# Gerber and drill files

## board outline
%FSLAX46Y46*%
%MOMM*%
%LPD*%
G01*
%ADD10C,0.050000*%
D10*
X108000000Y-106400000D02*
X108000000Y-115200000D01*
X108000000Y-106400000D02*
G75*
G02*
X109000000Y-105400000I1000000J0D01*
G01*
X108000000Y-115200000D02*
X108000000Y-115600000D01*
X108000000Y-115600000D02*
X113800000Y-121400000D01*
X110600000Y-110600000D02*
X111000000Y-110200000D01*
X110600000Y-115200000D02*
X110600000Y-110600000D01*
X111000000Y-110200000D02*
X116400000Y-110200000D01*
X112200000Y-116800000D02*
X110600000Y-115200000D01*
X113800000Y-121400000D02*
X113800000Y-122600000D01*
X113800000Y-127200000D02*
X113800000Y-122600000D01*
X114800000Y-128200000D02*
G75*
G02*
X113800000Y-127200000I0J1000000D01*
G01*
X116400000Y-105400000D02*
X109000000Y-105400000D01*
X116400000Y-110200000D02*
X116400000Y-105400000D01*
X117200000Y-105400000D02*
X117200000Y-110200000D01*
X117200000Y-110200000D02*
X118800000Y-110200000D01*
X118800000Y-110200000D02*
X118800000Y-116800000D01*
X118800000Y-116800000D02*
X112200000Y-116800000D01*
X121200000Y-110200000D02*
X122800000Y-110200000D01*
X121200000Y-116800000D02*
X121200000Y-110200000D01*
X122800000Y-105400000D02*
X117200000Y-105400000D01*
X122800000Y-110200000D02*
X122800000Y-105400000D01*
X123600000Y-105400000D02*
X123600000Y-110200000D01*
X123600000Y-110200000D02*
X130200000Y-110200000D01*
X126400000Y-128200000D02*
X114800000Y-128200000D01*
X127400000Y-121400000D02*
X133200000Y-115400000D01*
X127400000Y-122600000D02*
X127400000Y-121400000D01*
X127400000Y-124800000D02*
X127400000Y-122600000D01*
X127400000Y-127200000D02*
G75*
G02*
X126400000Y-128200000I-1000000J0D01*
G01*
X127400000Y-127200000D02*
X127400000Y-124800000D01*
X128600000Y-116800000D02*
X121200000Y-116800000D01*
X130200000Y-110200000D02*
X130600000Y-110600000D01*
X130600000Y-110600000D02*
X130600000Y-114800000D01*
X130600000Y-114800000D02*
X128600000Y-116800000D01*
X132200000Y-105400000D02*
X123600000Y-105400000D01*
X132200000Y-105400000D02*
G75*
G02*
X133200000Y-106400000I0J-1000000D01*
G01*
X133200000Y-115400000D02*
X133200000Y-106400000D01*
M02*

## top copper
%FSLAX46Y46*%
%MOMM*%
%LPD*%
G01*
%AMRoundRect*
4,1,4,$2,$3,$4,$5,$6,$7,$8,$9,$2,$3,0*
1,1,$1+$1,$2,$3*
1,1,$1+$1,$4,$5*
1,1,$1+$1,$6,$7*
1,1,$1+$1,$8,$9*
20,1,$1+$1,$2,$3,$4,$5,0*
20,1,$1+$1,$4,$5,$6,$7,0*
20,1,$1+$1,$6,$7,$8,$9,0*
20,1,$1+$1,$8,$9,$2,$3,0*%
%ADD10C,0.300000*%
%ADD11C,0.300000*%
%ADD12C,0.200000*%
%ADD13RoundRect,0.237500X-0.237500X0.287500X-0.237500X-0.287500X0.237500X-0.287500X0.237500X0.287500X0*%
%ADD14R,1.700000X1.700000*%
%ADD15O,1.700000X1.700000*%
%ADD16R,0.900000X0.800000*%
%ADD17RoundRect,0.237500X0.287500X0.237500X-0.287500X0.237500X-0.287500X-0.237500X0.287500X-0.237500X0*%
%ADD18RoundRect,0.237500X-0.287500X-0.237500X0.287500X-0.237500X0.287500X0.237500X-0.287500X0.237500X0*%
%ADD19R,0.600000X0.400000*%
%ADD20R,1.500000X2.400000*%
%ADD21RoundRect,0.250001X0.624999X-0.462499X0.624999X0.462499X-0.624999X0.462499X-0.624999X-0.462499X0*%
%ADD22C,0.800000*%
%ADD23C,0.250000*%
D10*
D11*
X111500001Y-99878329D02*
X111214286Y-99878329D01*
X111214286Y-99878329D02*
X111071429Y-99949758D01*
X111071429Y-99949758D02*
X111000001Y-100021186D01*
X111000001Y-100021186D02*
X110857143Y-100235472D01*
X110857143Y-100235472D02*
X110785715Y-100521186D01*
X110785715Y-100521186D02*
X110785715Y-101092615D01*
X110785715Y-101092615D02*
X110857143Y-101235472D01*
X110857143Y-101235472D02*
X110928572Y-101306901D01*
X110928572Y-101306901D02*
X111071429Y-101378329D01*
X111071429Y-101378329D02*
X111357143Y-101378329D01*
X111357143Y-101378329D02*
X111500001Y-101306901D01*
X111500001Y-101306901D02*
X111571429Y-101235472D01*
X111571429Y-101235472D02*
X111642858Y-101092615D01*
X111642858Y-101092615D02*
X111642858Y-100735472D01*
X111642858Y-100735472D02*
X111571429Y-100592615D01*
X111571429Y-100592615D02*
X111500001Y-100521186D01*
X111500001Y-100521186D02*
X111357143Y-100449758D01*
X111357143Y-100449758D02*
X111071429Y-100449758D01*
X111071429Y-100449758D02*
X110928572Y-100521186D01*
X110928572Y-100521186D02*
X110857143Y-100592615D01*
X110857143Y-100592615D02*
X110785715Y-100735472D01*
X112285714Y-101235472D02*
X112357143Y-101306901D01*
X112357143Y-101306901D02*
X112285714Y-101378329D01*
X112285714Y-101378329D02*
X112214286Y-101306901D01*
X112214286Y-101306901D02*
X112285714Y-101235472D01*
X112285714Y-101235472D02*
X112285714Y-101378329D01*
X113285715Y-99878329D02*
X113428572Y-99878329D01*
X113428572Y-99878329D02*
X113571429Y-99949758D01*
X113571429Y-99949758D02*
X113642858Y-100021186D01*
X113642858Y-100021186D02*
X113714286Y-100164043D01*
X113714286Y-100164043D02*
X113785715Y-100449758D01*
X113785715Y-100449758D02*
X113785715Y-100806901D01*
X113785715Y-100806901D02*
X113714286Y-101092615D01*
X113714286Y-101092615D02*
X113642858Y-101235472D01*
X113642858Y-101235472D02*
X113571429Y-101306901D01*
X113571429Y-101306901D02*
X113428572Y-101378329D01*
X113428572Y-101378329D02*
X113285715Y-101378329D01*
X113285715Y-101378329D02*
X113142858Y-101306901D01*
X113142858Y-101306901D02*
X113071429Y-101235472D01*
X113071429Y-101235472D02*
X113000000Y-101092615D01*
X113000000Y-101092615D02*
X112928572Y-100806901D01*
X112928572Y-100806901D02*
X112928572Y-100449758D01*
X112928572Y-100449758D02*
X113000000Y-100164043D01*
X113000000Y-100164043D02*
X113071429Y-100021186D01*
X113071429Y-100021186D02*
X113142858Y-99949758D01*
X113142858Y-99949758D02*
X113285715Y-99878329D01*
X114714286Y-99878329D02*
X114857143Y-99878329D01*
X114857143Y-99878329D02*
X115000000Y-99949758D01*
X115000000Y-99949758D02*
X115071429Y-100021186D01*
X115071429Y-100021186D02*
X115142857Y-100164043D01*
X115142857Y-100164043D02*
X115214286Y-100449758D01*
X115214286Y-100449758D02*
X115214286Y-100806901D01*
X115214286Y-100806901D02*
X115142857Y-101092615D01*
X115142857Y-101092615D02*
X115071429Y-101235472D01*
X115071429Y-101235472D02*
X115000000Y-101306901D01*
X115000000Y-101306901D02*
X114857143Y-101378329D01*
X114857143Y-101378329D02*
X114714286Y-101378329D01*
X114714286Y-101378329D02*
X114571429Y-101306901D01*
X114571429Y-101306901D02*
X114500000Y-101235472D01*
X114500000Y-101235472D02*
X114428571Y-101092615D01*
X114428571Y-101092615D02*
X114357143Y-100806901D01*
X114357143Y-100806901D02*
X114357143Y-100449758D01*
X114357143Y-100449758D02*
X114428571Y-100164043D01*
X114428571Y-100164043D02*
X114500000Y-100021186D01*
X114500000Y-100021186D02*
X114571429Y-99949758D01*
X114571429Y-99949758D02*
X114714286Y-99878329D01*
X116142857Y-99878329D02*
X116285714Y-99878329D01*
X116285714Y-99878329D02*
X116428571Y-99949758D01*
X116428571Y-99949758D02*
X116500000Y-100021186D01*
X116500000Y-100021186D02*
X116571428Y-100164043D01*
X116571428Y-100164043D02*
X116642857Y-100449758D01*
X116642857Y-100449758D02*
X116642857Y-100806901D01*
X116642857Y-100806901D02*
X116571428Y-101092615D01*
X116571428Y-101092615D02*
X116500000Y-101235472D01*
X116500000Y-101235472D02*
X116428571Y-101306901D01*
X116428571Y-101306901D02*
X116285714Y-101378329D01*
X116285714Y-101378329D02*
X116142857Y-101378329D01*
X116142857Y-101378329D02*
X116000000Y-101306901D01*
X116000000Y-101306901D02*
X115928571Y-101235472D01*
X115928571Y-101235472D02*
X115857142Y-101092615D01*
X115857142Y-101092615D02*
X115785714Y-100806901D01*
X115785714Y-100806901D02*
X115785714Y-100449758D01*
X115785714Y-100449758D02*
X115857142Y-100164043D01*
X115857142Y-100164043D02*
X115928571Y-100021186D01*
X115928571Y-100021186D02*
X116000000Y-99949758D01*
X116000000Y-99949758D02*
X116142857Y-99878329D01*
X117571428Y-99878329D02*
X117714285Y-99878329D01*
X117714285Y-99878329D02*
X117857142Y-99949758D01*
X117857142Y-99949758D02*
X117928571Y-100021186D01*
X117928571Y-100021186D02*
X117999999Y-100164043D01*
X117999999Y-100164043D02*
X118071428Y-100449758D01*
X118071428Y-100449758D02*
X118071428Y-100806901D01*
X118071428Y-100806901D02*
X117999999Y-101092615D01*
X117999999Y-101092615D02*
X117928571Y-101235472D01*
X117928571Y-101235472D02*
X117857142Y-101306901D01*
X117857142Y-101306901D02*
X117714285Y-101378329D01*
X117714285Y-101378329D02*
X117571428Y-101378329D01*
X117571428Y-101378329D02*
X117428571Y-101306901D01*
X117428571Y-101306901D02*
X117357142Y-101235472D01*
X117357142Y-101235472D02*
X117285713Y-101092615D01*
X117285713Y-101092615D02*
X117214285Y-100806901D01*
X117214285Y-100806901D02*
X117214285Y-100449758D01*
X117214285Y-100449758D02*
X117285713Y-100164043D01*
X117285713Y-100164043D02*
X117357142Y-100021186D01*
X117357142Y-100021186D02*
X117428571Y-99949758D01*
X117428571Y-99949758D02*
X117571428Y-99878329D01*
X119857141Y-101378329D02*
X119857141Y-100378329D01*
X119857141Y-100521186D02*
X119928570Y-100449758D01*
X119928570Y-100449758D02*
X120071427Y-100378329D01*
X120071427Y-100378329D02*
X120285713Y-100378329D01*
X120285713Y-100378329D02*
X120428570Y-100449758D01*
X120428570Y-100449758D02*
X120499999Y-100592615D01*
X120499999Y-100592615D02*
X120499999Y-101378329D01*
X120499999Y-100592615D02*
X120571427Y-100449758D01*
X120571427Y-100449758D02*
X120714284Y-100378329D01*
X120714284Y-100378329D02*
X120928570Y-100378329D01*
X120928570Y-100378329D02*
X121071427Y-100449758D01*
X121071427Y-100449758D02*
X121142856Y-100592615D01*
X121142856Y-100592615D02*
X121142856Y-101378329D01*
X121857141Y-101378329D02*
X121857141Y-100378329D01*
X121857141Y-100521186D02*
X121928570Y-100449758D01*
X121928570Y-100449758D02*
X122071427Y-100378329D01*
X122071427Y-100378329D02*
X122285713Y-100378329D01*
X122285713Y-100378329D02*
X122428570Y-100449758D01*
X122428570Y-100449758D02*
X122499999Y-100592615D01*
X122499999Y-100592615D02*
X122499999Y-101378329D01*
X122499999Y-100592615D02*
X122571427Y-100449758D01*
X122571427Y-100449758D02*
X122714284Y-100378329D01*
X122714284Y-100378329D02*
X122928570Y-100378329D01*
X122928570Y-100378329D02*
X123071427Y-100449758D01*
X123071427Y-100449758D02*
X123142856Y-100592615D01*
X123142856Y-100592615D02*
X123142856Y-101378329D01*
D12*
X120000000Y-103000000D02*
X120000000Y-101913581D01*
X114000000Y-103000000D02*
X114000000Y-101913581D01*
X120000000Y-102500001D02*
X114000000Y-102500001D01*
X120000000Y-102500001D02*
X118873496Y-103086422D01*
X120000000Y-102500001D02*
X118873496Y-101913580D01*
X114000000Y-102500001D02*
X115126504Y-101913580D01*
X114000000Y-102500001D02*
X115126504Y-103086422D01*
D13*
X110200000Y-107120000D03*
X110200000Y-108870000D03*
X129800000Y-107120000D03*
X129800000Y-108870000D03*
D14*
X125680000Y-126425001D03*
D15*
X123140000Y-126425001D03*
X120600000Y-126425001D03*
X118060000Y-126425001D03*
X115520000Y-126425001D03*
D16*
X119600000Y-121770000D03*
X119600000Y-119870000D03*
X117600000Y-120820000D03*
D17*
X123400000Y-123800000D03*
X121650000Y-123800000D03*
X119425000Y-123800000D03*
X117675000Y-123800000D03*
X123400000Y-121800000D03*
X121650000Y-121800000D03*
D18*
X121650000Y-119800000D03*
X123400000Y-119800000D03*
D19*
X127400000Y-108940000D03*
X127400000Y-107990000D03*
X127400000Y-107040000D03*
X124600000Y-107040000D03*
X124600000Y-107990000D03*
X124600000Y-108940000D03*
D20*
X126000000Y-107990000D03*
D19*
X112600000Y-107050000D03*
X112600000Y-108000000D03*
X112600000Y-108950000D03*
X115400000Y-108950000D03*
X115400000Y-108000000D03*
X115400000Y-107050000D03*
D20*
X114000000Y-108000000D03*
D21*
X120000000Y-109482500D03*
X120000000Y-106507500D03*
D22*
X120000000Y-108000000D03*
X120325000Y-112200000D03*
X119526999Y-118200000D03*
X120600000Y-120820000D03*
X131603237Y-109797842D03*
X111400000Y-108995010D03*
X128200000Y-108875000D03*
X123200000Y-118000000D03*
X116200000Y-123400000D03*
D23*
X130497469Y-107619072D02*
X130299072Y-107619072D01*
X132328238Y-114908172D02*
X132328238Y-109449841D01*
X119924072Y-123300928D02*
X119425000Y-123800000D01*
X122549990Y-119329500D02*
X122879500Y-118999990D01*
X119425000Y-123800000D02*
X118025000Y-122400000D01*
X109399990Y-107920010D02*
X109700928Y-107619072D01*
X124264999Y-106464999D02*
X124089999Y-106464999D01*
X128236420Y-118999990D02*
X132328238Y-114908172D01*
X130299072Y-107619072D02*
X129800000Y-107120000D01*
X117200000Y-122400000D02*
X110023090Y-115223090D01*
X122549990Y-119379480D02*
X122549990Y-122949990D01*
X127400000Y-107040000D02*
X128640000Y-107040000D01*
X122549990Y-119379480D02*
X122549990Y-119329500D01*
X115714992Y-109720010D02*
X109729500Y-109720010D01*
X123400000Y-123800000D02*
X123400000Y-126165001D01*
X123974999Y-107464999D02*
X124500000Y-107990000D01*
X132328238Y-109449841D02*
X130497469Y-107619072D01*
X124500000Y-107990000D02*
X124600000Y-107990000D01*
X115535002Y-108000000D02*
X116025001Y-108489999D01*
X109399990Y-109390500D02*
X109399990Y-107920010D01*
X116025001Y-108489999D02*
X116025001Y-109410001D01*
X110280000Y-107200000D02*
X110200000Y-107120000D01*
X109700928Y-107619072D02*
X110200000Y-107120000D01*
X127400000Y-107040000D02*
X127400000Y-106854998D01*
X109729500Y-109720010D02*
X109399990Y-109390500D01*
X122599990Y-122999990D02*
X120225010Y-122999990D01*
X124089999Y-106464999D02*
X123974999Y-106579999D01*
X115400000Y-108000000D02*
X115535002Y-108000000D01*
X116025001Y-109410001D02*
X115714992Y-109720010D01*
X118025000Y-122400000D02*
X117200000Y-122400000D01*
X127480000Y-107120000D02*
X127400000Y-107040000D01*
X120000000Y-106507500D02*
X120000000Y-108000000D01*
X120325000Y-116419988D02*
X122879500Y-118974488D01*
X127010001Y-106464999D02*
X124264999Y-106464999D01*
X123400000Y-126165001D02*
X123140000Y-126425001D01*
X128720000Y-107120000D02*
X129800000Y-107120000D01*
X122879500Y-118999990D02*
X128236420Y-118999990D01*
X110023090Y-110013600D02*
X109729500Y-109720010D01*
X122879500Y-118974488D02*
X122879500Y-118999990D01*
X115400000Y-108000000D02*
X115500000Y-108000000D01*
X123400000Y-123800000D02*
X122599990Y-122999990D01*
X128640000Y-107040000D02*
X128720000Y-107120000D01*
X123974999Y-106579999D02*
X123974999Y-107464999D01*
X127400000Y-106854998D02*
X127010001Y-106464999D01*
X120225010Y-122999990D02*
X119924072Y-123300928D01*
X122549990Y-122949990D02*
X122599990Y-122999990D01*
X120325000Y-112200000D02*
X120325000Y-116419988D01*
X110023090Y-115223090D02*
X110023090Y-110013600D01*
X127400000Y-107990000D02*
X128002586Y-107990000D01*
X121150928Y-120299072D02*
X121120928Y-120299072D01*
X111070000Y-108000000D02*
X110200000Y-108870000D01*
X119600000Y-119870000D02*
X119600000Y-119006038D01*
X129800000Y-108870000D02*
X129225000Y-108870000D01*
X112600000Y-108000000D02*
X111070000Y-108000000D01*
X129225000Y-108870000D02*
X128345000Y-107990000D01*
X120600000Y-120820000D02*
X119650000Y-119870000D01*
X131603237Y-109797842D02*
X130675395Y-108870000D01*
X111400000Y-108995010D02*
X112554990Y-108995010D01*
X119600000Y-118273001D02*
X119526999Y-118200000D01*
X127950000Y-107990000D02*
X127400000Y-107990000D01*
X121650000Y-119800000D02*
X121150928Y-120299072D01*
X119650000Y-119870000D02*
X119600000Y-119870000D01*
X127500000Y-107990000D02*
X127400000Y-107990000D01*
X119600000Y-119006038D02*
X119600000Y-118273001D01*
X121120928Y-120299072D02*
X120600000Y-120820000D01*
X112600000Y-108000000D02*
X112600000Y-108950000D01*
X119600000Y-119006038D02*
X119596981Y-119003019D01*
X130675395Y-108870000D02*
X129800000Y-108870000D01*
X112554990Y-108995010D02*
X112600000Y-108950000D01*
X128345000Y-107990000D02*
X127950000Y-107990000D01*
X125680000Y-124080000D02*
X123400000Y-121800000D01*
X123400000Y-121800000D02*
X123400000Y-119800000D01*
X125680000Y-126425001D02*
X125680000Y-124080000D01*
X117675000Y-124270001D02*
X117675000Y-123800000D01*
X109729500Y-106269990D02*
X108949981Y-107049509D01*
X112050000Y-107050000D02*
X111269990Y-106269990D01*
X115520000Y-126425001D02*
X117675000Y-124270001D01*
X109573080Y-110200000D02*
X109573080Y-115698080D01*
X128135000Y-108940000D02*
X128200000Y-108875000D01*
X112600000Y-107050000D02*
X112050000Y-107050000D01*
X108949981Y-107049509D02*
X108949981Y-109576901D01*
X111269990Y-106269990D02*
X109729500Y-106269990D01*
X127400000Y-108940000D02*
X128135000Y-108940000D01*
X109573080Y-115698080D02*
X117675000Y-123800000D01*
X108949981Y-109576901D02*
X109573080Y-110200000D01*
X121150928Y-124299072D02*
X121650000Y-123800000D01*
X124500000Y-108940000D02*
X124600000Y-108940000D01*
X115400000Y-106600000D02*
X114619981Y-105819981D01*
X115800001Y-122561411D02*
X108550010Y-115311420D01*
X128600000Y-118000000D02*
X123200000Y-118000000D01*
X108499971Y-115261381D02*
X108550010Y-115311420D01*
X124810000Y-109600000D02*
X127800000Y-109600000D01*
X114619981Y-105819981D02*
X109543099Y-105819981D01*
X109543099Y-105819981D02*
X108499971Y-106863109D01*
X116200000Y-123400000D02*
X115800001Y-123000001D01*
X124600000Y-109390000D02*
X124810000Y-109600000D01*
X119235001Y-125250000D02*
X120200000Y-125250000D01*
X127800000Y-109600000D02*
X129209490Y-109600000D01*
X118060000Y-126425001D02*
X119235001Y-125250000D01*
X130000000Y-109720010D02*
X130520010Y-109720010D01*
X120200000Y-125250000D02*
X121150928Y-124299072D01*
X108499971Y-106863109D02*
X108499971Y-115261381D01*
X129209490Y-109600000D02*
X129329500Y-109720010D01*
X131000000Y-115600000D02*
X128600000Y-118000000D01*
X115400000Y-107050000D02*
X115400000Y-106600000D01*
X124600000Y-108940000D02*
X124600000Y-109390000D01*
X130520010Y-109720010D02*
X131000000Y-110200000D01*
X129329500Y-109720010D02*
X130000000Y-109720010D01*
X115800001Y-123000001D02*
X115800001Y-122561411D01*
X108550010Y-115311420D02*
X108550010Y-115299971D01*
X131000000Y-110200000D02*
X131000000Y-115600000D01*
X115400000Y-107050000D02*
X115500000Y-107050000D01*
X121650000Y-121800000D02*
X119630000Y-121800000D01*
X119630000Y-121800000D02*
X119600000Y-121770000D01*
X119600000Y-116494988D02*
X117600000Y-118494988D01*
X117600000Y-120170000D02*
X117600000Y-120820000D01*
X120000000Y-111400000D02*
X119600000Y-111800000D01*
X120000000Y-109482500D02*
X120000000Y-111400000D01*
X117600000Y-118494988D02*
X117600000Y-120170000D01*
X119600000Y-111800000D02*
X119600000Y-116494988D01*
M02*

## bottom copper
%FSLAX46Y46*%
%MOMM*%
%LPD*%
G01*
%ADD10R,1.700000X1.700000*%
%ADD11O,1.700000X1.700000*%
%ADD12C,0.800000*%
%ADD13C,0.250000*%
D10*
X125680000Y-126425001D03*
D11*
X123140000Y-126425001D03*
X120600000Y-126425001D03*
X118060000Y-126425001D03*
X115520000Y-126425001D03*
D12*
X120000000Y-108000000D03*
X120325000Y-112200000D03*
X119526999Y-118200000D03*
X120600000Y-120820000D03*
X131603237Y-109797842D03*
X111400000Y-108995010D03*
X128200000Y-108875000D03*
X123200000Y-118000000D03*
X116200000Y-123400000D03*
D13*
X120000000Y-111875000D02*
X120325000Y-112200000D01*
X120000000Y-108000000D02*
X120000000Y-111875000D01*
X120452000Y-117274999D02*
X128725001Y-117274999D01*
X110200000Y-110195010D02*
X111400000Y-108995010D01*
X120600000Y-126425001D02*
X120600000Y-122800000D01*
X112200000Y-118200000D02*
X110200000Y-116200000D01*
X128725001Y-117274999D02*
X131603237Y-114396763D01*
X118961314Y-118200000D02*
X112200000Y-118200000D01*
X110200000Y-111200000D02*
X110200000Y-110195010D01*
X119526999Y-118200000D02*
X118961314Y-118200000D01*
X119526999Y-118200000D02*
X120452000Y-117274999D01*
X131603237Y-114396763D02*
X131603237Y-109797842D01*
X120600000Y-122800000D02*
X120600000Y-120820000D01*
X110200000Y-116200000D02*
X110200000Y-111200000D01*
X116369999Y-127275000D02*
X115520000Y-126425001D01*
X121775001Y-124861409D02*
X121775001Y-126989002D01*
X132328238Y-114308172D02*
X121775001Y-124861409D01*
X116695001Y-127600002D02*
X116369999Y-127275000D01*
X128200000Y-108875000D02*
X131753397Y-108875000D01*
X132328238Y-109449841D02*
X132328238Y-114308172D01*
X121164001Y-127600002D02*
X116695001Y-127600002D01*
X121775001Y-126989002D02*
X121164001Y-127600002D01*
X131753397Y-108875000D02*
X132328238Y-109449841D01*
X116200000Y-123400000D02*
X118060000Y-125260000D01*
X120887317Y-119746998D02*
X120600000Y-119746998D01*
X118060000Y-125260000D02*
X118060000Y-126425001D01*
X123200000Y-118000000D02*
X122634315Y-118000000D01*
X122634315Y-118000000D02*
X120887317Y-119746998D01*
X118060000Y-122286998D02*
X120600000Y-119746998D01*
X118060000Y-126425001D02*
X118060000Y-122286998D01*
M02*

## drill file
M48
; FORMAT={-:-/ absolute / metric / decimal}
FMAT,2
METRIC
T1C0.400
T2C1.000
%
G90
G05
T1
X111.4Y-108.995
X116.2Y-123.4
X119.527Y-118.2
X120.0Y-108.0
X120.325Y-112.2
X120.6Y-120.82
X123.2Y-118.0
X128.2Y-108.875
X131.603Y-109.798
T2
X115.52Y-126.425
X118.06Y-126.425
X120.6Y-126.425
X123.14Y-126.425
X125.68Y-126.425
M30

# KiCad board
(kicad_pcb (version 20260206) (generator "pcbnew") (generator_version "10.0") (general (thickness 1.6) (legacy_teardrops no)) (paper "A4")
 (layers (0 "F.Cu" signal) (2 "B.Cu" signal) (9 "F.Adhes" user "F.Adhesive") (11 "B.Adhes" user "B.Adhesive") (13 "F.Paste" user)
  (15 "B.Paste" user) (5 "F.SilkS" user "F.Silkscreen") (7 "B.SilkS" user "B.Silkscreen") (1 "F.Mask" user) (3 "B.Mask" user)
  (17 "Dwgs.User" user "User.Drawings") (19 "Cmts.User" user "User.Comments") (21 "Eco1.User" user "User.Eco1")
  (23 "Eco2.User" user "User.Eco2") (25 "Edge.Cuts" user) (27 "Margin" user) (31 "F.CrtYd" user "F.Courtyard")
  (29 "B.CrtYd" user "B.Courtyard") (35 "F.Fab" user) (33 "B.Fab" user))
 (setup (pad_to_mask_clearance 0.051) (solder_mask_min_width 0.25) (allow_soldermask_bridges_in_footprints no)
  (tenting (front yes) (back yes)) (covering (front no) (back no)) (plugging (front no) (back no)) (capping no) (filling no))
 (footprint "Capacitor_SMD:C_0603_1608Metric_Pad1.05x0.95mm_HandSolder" (layer "F.Cu") (at 110.2 107.995 -90)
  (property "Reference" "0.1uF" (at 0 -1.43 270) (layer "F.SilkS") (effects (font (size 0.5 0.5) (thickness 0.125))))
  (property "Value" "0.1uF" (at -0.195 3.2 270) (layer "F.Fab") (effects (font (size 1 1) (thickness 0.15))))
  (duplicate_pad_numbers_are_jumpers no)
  (pad "1" smd roundrect (at -0.875 0 270) (size 1.05 0.95) (layers "F.Cu" "F.Mask" "F.Paste") (roundrect_rratio 0.25) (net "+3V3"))
  (pad "2" smd roundrect (at 0.875 0 270) (size 1.05 0.95) (layers "F.Cu" "F.Mask" "F.Paste") (roundrect_rratio 0.25) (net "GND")))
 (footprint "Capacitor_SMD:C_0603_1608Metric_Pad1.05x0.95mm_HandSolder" (layer "F.Cu") (at 129.8 107.995 -90)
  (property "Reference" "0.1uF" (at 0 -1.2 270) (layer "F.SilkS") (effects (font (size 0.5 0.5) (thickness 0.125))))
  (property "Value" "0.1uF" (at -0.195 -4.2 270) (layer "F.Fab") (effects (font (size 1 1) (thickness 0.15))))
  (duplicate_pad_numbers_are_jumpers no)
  (pad "1" smd roundrect (at -0.875 0 270) (size 1.05 0.95) (layers "F.Cu" "F.Mask" "F.Paste") (roundrect_rratio 0.25) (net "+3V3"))
  (pad "2" smd roundrect (at 0.875 0 270) (size 1.05 0.95) (layers "F.Cu" "F.Mask" "F.Paste") (roundrect_rratio 0.25) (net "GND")))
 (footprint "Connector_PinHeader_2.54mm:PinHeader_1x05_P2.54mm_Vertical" (layer "F.Cu") (at 125.68 126.425001 -90)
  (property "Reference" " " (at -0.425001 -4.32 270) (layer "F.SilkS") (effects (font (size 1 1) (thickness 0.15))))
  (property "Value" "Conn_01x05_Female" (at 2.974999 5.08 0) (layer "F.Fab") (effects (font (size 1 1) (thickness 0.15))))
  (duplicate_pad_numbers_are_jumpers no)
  (pad "1" thru_hole rect (at 0 0 270) (size 1.7 1.7) (drill 1) (layers "*.Cu" "*.Mask") (remove_unused_layers no) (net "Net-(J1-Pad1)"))
  (pad "2" thru_hole oval (at 0 2.54 270) (size 1.7 1.7) (drill 1) (layers "*.Cu" "*.Mask") (remove_unused_layers no) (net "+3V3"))
  (pad "3" thru_hole oval (at 0 5.08 270) (size 1.7 1.7) (drill 1) (layers "*.Cu" "*.Mask") (remove_unused_layers no) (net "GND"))
  (pad "4" thru_hole oval (at 0 7.62 270) (size 1.7 1.7) (drill 1) (layers "*.Cu" "*.Mask") (remove_unused_layers no) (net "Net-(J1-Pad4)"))
  (pad "5" thru_hole oval (at 0 10.16 270) (size 1.7 1.7) (drill 1) (layers "*.Cu" "*.Mask") (remove_unused_layers no) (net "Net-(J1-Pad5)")))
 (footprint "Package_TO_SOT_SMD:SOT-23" (layer "F.Cu") (at 118.6 120.82 180)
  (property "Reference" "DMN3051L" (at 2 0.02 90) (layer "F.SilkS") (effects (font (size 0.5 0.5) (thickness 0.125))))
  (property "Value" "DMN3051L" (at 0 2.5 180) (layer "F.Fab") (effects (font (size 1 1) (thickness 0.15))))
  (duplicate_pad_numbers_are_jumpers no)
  (pad "1" smd rect (at -1 -0.95 180) (size 0.9 0.8) (layers "F.Cu" "F.Mask" "F.Paste") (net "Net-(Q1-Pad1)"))
  (pad "2" smd rect (at -1 0.95 180) (size 0.9 0.8) (layers "F.Cu" "F.Mask" "F.Paste") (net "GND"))
  (pad "3" smd rect (at 1 0 180) (size 0.9 0.8) (layers "F.Cu" "F.Mask" "F.Paste") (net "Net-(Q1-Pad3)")))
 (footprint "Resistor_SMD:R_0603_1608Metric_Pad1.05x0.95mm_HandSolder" (layer "F.Cu") (at 122.525 123.8 180)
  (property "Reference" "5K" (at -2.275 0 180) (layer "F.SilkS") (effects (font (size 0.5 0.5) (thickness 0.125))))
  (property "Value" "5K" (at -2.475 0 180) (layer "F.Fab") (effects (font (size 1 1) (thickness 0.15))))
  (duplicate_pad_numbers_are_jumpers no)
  (pad "1" smd roundrect (at -0.875 0 180) (size 1.05 0.95) (layers "F.Cu" "F.Mask" "F.Paste") (roundrect_rratio 0.25) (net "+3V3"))
  (pad "2" smd roundrect (at 0.875 0 180) (size 1.05 0.95) (layers "F.Cu" "F.Mask" "F.Paste") (roundrect_rratio 0.25) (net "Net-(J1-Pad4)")))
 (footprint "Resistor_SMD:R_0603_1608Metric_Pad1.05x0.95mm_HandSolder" (layer "F.Cu") (at 118.55 123.8 180)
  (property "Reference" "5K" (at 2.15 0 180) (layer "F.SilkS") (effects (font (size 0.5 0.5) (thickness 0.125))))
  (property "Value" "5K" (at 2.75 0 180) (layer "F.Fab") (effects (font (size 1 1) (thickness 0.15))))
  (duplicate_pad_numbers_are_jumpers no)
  (pad "1" smd roundrect (at -0.875 0 180) (size 1.05 0.95) (layers "F.Cu" "F.Mask" "F.Paste") (roundrect_rratio 0.25) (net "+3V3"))
  (pad "2" smd roundrect (at 0.875 0 180) (size 1.05 0.95) (layers "F.Cu" "F.Mask" "F.Paste") (roundrect_rratio 0.25) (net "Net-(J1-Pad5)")))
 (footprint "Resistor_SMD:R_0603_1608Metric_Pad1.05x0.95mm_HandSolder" (layer "F.Cu") (at 122.525 121.8 180)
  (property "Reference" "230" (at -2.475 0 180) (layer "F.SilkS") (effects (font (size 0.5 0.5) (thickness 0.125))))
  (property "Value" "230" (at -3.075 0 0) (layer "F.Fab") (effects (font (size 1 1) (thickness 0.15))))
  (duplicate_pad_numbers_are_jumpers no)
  (pad "1" smd roundrect (at -0.875 0 180) (size 1.05 0.95) (layers "F.Cu" "F.Mask" "F.Paste") (roundrect_rratio 0.25) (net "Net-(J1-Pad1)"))
  (pad "2" smd roundrect (at 0.875 0 180) (size 1.05 0.95) (layers "F.Cu" "F.Mask" "F.Paste") (roundrect_rratio 0.25) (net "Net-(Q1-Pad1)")))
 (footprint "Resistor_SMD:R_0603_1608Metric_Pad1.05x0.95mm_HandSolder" (layer "F.Cu") (at 122.525 119.8)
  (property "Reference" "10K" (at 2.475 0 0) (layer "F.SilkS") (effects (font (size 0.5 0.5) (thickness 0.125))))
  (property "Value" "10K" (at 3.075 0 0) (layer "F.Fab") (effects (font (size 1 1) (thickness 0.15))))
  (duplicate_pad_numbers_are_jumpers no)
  (pad "1" smd roundrect (at -0.875 0) (size 1.05 0.95) (layers "F.Cu" "F.Mask" "F.Paste") (roundrect_rratio 0.25) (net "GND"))
  (pad "2" smd roundrect (at 0.875 0) (size 1.05 0.95) (layers "F.Cu" "F.Mask" "F.Paste") (roundrect_rratio 0.25) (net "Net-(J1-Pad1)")))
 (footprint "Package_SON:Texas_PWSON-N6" (layer "F.Cu") (at 126 107.99 180)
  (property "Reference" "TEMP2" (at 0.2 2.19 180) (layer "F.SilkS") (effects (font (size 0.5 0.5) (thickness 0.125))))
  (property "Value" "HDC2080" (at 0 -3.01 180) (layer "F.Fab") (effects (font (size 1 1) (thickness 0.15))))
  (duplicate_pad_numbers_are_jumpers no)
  (pad "1" smd rect (at -1.4 -0.95 180) (size 0.6 0.4) (layers "F.Cu" "F.Mask" "F.Paste") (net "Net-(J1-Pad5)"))
  (pad "2" smd rect (at -1.4 0 180) (size 0.6 0.4) (layers "F.Cu" "F.Mask" "F.Paste") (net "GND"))
  (pad "3" smd rect (at -1.4 0.95 180) (size 0.6 0.4) (layers "F.Cu" "F.Mask" "F.Paste") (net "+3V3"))
  (pad "4" smd rect (at 1.4 0.95 180) (size 0.6 0.4) (layers "F.Cu" "F.Mask" "F.Paste") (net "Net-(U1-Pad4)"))
  (pad "5" smd rect (at 1.4 0 180) (size 0.6 0.4) (layers "F.Cu" "F.Mask" "F.Paste") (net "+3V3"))
  (pad "6" smd rect (at 1.4 -0.95 180) (size 0.6 0.4) (layers "F.Cu" "F.Mask" "F.Paste") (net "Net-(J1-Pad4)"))
  (pad "7" smd rect (at 0 0 180) (size 1.5 2.4) (layers "F.Cu" "F.Mask" "F.Paste") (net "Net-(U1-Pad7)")))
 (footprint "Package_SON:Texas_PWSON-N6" (layer "F.Cu") (at 114 108)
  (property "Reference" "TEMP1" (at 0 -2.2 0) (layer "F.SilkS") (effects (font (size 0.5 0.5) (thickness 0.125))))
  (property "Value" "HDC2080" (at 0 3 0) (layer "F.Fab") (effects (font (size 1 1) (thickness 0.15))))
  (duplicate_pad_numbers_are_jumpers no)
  (pad "1" smd rect (at -1.4 -0.95) (size 0.6 0.4) (layers "F.Cu" "F.Mask" "F.Paste") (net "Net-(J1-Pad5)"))
  (pad "2" smd rect (at -1.4 0) (size 0.6 0.4) (layers "F.Cu" "F.Mask" "F.Paste") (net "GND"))
  (pad "3" smd rect (at -1.4 0.95) (size 0.6 0.4) (layers "F.Cu" "F.Mask" "F.Paste") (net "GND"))
  (pad "4" smd rect (at 1.4 0.95) (size 0.6 0.4) (layers "F.Cu" "F.Mask" "F.Paste") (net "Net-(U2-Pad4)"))
  (pad "5" smd rect (at 1.4 0) (size 0.6 0.4) (layers "F.Cu" "F.Mask" "F.Paste") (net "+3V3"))
  (pad "6" smd rect (at 1.4 -0.95) (size 0.6 0.4) (layers "F.Cu" "F.Mask" "F.Paste") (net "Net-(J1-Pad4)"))
  (pad "7" smd rect (at 0 0) (size 1.5 2.4) (layers "F.Cu" "F.Mask" "F.Paste") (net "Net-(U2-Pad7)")))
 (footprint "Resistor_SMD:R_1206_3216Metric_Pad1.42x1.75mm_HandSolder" (layer "F.Cu") (at 120 107.995 90)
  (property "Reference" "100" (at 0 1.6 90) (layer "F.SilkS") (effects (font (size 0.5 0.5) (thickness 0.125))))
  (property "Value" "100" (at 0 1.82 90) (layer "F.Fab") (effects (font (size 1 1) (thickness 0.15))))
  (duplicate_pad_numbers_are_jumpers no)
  (pad "1" smd roundrect (at -1.4875 0 90) (size 1.425 1.75) (layers "F.Cu" "F.Mask" "F.Paste") (roundrect_rratio 0.175439)
   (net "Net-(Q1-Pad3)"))
  (pad "2" smd roundrect (at 1.4875 0 90) (size 1.425 1.75) (layers "F.Cu" "F.Mask" "F.Paste") (roundrect_rratio 0.175439) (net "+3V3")))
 (gr_line (start 108 106.4) (end 108 115.2) (stroke (width 0.05) (type solid)) (layer "Edge.Cuts"))
 (gr_arc (start 108 106.4) (mid 108.292893 105.692893) (end 109 105.4) (stroke (width 0.05) (type solid)) (layer "Edge.Cuts"))
 (gr_line (start 108 115.2) (end 108 115.6) (stroke (width 0.05) (type solid)) (layer "Edge.Cuts"))
 (gr_line (start 108 115.6) (end 113.8 121.4) (stroke (width 0.05) (type solid)) (layer "Edge.Cuts"))
 (gr_line (start 110.6 110.6) (end 111 110.2) (stroke (width 0.05) (type solid)) (layer "Edge.Cuts"))
 (gr_line (start 110.6 115.2) (end 110.6 110.6) (stroke (width 0.05) (type solid)) (layer "Edge.Cuts"))
 (gr_line (start 111 110.2) (end 116.4 110.2) (stroke (width 0.05) (type solid)) (layer "Edge.Cuts"))
 (gr_line (start 112.2 116.8) (end 110.6 115.2) (stroke (width 0.05) (type solid)) (layer "Edge.Cuts"))
 (gr_line (start 113.8 121.4) (end 113.8 122.6) (stroke (width 0.05) (type solid)) (layer "Edge.Cuts"))
 (gr_line (start 113.8 127.2) (end 113.8 122.6) (stroke (width 0.05) (type solid)) (layer "Edge.Cuts"))
 (gr_arc (start 114.8 128.2) (mid 114.092893 127.907107) (end 113.8 127.2) (stroke (width 0.05) (type solid)) (layer "Edge.Cuts"))
 (gr_line (start 116.4 105.4) (end 109 105.4) (stroke (width 0.05) (type solid)) (layer "Edge.Cuts"))
 (gr_line (start 116.4 110.2) (end 116.4 105.4) (stroke (width 0.05) (type solid)) (layer "Edge.Cuts"))
 (gr_line (start 117.2 105.4) (end 117.2 110.2) (stroke (width 0.05) (type solid)) (layer "Edge.Cuts"))
 (gr_line (start 117.2 110.2) (end 118.8 110.2) (stroke (width 0.05) (type solid)) (layer "Edge.Cuts"))
 (gr_line (start 118.8 110.2) (end 118.8 116.8) (stroke (width 0.05) (type solid)) (layer "Edge.Cuts"))
 (gr_line (start 118.8 116.8) (end 112.2 116.8) (stroke (width 0.05) (type solid)) (layer "Edge.Cuts"))
 (gr_line (start 121.2 110.2) (end 122.8 110.2) (stroke (width 0.05) (type solid)) (layer "Edge.Cuts"))
 (gr_line (start 121.2 116.8) (end 121.2 110.2) (stroke (width 0.05) (type solid)) (layer "Edge.Cuts"))
 (gr_line (start 122.8 105.4) (end 117.2 105.4) (stroke (width 0.05) (type solid)) (layer "Edge.Cuts"))
 (gr_line (start 122.8 110.2) (end 122.8 105.4) (stroke (width 0.05) (type solid)) (layer "Edge.Cuts"))
 (gr_line (start 123.6 105.4) (end 123.6 110.2) (stroke (width 0.05) (type solid)) (layer "Edge.Cuts"))
 (gr_line (start 123.6 110.2) (end 130.2 110.2) (stroke (width 0.05) (type solid)) (layer "Edge.Cuts"))
 (gr_line (start 126.4 128.2) (end 114.8 128.2) (stroke (width 0.05) (type solid)) (layer "Edge.Cuts"))
 (gr_line (start 127.4 121.4) (end 133.2 115.4) (stroke (width 0.05) (type solid)) (layer "Edge.Cuts"))
 (gr_line (start 127.4 122.6) (end 127.4 121.4) (stroke (width 0.05) (type solid)) (layer "Edge.Cuts"))
 (gr_line (start 127.4 124.8) (end 127.4 122.6) (stroke (width 0.05) (type solid)) (layer "Edge.Cuts"))
 (gr_arc (start 127.4 127.2) (mid 127.107107 127.907107) (end 126.4 128.2) (stroke (width 0.05) (type solid)) (layer "Edge.Cuts"))
 (gr_line (start 127.4 127.2) (end 127.4 124.8) (stroke (width 0.05) (type solid)) (layer "Edge.Cuts"))
 (gr_line (start 128.6 116.8) (end 121.2 116.8) (stroke (width 0.05) (type solid)) (layer "Edge.Cuts"))
 (gr_line (start 130.2 110.2) (end 130.6 110.6) (stroke (width 0.05) (type solid)) (layer "Edge.Cuts"))
 (gr_line (start 130.6 110.6) (end 130.6 114.8) (stroke (width 0.05) (type solid)) (layer "Edge.Cuts"))
 (gr_line (start 130.6 114.8) (end 128.6 116.8) (stroke (width 0.05) (type solid)) (layer "Edge.Cuts"))
 (gr_line (start 132.2 105.4) (end 123.6 105.4) (stroke (width 0.05) (type solid)) (layer "Edge.Cuts"))
 (gr_arc (start 132.2 105.4) (mid 132.907107 105.692893) (end 133.2 106.4) (stroke (width 0.05) (type solid)) (layer "Edge.Cuts"))
 (gr_line (start 133.2 115.4) (end 133.2 106.4) (stroke (width 0.05) (type solid)) (layer "Edge.Cuts"))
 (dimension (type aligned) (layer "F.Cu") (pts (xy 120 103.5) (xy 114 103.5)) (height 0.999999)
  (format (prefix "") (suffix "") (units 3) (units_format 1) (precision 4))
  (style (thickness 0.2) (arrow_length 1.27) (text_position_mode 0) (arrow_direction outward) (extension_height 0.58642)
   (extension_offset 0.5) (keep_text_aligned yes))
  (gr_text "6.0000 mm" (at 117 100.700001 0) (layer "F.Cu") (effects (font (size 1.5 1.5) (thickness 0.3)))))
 (segment (start 130.497469 107.619072) (end 130.299072 107.619072) (width 0.25) (layer "F.Cu") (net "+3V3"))
 (segment (start 132.328238 114.908172) (end 132.328238 109.449841) (width 0.25) (layer "F.Cu") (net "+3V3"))
 (segment (start 119.924072 123.300928) (end 119.425 123.8) (width 0.25) (layer "F.Cu") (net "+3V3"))
 (segment (start 122.54999 119.3295) (end 122.8795 118.99999) (width 0.25) (layer "F.Cu") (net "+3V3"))
 (segment (start 119.425 123.8) (end 118.025 122.4) (width 0.25) (layer "F.Cu") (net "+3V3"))
 (segment (start 109.39999 107.92001) (end 109.700928 107.619072) (width 0.25) (layer "F.Cu") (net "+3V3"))
 (segment (start 124.264999 106.464999) (end 124.089999 106.464999) (width 0.25) (layer "F.Cu") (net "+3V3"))
 (segment (start 128.23642 118.99999) (end 132.328238 114.908172) (width 0.25) (layer "F.Cu") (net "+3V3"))
 (segment (start 130.299072 107.619072) (end 129.8 107.12) (width 0.25) (layer "F.Cu") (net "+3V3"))
 (segment (start 117.2 122.4) (end 110.02309 115.22309) (width 0.25) (layer "F.Cu") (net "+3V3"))
 (segment (start 122.54999 119.37948) (end 122.54999 122.94999) (width 0.25) (layer "F.Cu") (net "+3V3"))
 (segment (start 127.4 107.04) (end 128.64 107.04) (width 0.25) (layer "F.Cu") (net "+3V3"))
 (segment (start 122.54999 119.37948) (end 122.54999 119.3295) (width 0.25) (layer "F.Cu") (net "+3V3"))
 (segment (start 115.714992 109.72001) (end 109.7295 109.72001) (width 0.25) (layer "F.Cu") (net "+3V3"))
 (segment (start 123.4 123.8) (end 123.4 126.165001) (width 0.25) (layer "F.Cu") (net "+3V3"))
 (segment (start 123.974999 107.464999) (end 124.5 107.99) (width 0.25) (layer "F.Cu") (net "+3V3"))
 (segment (start 132.328238 109.449841) (end 130.497469 107.619072) (width 0.25) (layer "F.Cu") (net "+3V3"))
 (segment (start 124.5 107.99) (end 124.6 107.99) (width 0.25) (layer "F.Cu") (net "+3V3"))
 (segment (start 115.535002 108) (end 116.025001 108.489999) (width 0.25) (layer "F.Cu") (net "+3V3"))
 (segment (start 109.39999 109.3905) (end 109.39999 107.92001) (width 0.25) (layer "F.Cu") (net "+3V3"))
 (segment (start 116.025001 108.489999) (end 116.025001 109.410001) (width 0.25) (layer "F.Cu") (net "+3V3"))
 (segment (start 110.28 107.2) (end 110.2 107.12) (width 0.25) (layer "F.Cu") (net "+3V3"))
 (segment (start 109.700928 107.619072) (end 110.2 107.12) (width 0.25) (layer "F.Cu") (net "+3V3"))
 (segment (start 127.4 107.04) (end 127.4 106.854998) (width 0.25) (layer "F.Cu") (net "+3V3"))
 (segment (start 109.7295 109.72001) (end 109.39999 109.3905) (width 0.25) (layer "F.Cu") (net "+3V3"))
 (segment (start 122.59999 122.99999) (end 120.22501 122.99999) (width 0.25) (layer "F.Cu") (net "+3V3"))
 (segment (start 124.089999 106.464999) (end 123.974999 106.579999) (width 0.25) (layer "F.Cu") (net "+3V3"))
 (segment (start 115.4 108) (end 115.535002 108) (width 0.25) (layer "F.Cu") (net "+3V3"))
 (segment (start 116.025001 109.410001) (end 115.714992 109.72001) (width 0.25) (layer "F.Cu") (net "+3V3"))
 (segment (start 118.025 122.4) (end 117.2 122.4) (width 0.25) (layer "F.Cu") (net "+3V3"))
 (segment (start 127.48 107.12) (end 127.4 107.04) (width 0.25) (layer "F.Cu") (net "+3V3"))
 (segment (start 120 106.5075) (end 120 108) (width 0.25) (layer "F.Cu") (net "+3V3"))
 (segment (start 120.325 116.419988) (end 122.8795 118.974488) (width 0.25) (layer "F.Cu") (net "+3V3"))
 (segment (start 127.010001 106.464999) (end 124.264999 106.464999) (width 0.25) (layer "F.Cu") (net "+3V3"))
 (segment (start 123.4 126.165001) (end 123.14 126.425001) (width 0.25) (layer "F.Cu") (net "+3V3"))
 (segment (start 128.72 107.12) (end 129.8 107.12) (width 0.25) (layer "F.Cu") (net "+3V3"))
 (segment (start 122.8795 118.99999) (end 128.23642 118.99999) (width 0.25) (layer "F.Cu") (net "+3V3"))
 (segment (start 110.02309 110.0136) (end 109.7295 109.72001) (width 0.25) (layer "F.Cu") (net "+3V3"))
 (segment (start 122.8795 118.974488) (end 122.8795 118.99999) (width 0.25) (layer "F.Cu") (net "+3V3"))
 (segment (start 115.4 108) (end 115.5 108) (width 0.25) (layer "F.Cu") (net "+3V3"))
 (segment (start 123.4 123.8) (end 122.59999 122.99999) (width 0.25) (layer "F.Cu") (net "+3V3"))
 (segment (start 128.64 107.04) (end 128.72 107.12) (width 0.25) (layer "F.Cu") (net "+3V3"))
 (segment (start 123.974999 106.579999) (end 123.974999 107.464999) (width 0.25) (layer "F.Cu") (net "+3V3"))
 (segment (start 127.4 106.854998) (end 127.010001 106.464999) (width 0.25) (layer "F.Cu") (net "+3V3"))
 (segment (start 120.22501 122.99999) (end 119.924072 123.300928) (width 0.25) (layer "F.Cu") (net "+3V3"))
 (segment (start 122.54999 122.94999) (end 122.59999 122.99999) (width 0.25) (layer "F.Cu") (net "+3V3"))
 (segment (start 120.325 112.2) (end 120.325 116.419988) (width 0.25) (layer "F.Cu") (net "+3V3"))
 (segment (start 110.02309 115.22309) (end 110.02309 110.0136) (width 0.25) (layer "F.Cu") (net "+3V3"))
 (via (at 120 108) (size 0.8) (drill 0.4) (layers "F.Cu" "B.Cu") (capping no) (covering (front no) (back no))
  (plugging (front no) (back no)) (filling no) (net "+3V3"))
 (via (at 120.325 112.2) (size 0.8) (drill 0.4) (layers "F.Cu" "B.Cu") (capping no) (covering (front no) (back no))
  (plugging (front no) (back no)) (filling no) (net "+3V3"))
 (segment (start 120 111.875) (end 120.325 112.2) (width 0.25) (layer "B.Cu") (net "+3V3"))
 (segment (start 120 108) (end 120 111.875) (width 0.25) (layer "B.Cu") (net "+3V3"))
 (segment (start 127.4 107.99) (end 128.002586 107.99) (width 0.25) (layer "F.Cu") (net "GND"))
 (segment (start 121.150928 120.299072) (end 121.120928 120.299072) (width 0.25) (layer "F.Cu") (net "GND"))
 (segment (start 111.07 108) (end 110.2 108.87) (width 0.25) (layer "F.Cu") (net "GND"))
 (segment (start 119.6 119.87) (end 119.6 119.006038) (width 0.25) (layer "F.Cu") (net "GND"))
 (segment (start 129.8 108.87) (end 129.225 108.87) (width 0.25) (layer "F.Cu") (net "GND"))
 (segment (start 112.6 108) (end 111.07 108) (width 0.25) (layer "F.Cu") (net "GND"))
 (segment (start 129.225 108.87) (end 128.345 107.99) (width 0.25) (layer "F.Cu") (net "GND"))
 (segment (start 120.6 120.82) (end 119.65 119.87) (width 0.25) (layer "F.Cu") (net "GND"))
 (segment (start 131.603237 109.797842) (end 130.675395 108.87) (width 0.25) (layer "F.Cu") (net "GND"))
 (segment (start 111.4 108.99501) (end 112.55499 108.99501) (width 0.25) (layer "F.Cu") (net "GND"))
 (segment (start 119.6 118.273001) (end 119.526999 118.2) (width 0.25) (layer "F.Cu") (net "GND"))
 (segment (start 127.95 107.99) (end 127.4 107.99) (width 0.25) (layer "F.Cu") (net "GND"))
 (segment (start 121.65 119.8) (end 121.150928 120.299072) (width 0.25) (layer "F.Cu") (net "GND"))
 (segment (start 119.65 119.87) (end 119.6 119.87) (width 0.25) (layer "F.Cu") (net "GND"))
 (segment (start 127.5 107.99) (end 127.4 107.99) (width 0.25) (layer "F.Cu") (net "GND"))
 (segment (start 119.6 119.006038) (end 119.6 118.273001) (width 0.25) (layer "F.Cu") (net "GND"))
 (segment (start 121.120928 120.299072) (end 120.6 120.82) (width 0.25) (layer "F.Cu") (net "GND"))
 (segment (start 112.6 108) (end 112.6 108.95) (width 0.25) (layer "F.Cu") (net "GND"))
 (segment (start 119.6 119.006038) (end 119.596981 119.003019) (width 0.25) (layer "F.Cu") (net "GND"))
 (segment (start 130.675395 108.87) (end 129.8 108.87) (width 0.25) (layer "F.Cu") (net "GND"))
 (segment (start 112.55499 108.99501) (end 112.6 108.95) (width 0.25) (layer "F.Cu") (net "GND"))
 (segment (start 128.345 107.99) (end 127.95 107.99) (width 0.25) (layer "F.Cu") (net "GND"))
 (via (at 119.526999 118.2) (size 0.8) (drill 0.4) (layers "F.Cu" "B.Cu") (capping no) (covering (front no) (back no))
  (plugging (front no) (back no)) (filling no) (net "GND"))
 (via (at 120.6 120.82) (size 0.8) (drill 0.4) (layers "F.Cu" "B.Cu") (capping no) (covering (front no) (back no))
  (plugging (front no) (back no)) (filling no) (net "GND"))
 (via (at 131.603237 109.797842) (size 0.8) (drill 0.4) (layers "F.Cu" "B.Cu") (capping no) (covering (front no) (back no))
  (plugging (front no) (back no)) (filling no) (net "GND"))
 (via (at 111.4 108.99501) (size 0.8) (drill 0.4) (layers "F.Cu" "B.Cu") (capping no) (covering (front no) (back no))
  (plugging (front no) (back no)) (filling no) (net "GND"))
 (segment (start 120.452 117.274999) (end 128.725001 117.274999) (width 0.25) (layer "B.Cu") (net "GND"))
 (segment (start 110.2 110.19501) (end 111.4 108.99501) (width 0.25) (layer "B.Cu") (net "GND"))
 (segment (start 120.6 126.425001) (end 120.6 122.8) (width 0.25) (layer "B.Cu") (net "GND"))
 (segment (start 112.2 118.2) (end 110.2 116.2) (width 0.25) (layer "B.Cu") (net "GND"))
 (segment (start 128.725001 117.274999) (end 131.603237 114.396763) (width 0.25) (layer "B.Cu") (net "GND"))
 (segment (start 118.961314 118.2) (end 112.2 118.2) (width 0.25) (layer "B.Cu") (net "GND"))
 (segment (start 110.2 111.2) (end 110.2 110.19501) (width 0.25) (layer "B.Cu") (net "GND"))
 (segment (start 119.526999 118.2) (end 118.961314 118.2) (width 0.25) (layer "B.Cu") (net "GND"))
 (segment (start 119.526999 118.2) (end 120.452 117.274999) (width 0.25) (layer "B.Cu") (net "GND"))
 (segment (start 131.603237 114.396763) (end 131.603237 109.797842) (width 0.25) (layer "B.Cu") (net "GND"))
 (segment (start 120.6 122.8) (end 120.6 120.82) (width 0.25) (layer "B.Cu") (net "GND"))
 (segment (start 110.2 116.2) (end 110.2 111.2) (width 0.25) (layer "B.Cu") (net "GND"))
 (segment (start 125.68 124.08) (end 123.4 121.8) (width 0.25) (layer "F.Cu") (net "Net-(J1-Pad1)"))
 (segment (start 123.4 121.8) (end 123.4 119.8) (width 0.25) (layer "F.Cu") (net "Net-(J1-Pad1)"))
 (segment (start 125.68 126.425001) (end 125.68 124.08) (width 0.25) (layer "F.Cu") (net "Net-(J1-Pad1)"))
 (segment (start 117.675 124.270001) (end 117.675 123.8) (width 0.25) (layer "F.Cu") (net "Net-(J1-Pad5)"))
 (segment (start 109.7295 106.26999) (end 108.949981 107.049509) (width 0.25) (layer "F.Cu") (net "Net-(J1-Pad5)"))
 (segment (start 112.05 107.05) (end 111.26999 106.26999) (width 0.25) (layer "F.Cu") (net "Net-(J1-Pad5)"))
 (segment (start 115.52 126.425001) (end 117.675 124.270001) (width 0.25) (layer "F.Cu") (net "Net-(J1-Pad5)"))
 (segment (start 109.57308 110.2) (end 109.57308 115.69808) (width 0.25) (layer "F.Cu") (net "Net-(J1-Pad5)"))
 (segment (start 128.135 108.94) (end 128.2 108.875) (width 0.25) (layer "F.Cu") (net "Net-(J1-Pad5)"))
 (segment (start 112.6 107.05) (end 112.05 107.05) (width 0.25) (layer "F.Cu") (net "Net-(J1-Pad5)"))
 (segment (start 108.949981 107.049509) (end 108.949981 109.576901) (width 0.25) (layer "F.Cu") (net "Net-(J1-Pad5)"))
 (segment (start 111.26999 106.26999) (end 109.7295 106.26999) (width 0.25) (layer "F.Cu") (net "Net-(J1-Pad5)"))
 (segment (start 127.4 108.94) (end 128.135 108.94) (width 0.25) (layer "F.Cu") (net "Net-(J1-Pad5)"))
 (segment (start 109.57308 115.69808) (end 117.675 123.8) (width 0.25) (layer "F.Cu") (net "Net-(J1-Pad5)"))
 (segment (start 108.949981 109.576901) (end 109.57308 110.2) (width 0.25) (layer "F.Cu") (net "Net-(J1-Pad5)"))
 (via (at 128.2 108.875) (size 0.8) (drill 0.4) (layers "F.Cu" "B.Cu") (capping no) (covering (front no) (back no))
  (plugging (front no) (back no)) (filling no) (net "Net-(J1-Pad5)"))
 (segment (start 116.369999 127.275) (end 115.52 126.425001) (width 0.25) (layer "B.Cu") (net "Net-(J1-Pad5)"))
 (segment (start 121.775001 124.861409) (end 121.775001 126.989002) (width 0.25) (layer "B.Cu") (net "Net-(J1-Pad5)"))
 (segment (start 132.328238 114.308172) (end 121.775001 124.861409) (width 0.25) (layer "B.Cu") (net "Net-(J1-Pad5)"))
 (segment (start 116.695001 127.600002) (end 116.369999 127.275) (width 0.25) (layer "B.Cu") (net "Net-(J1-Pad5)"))
 (segment (start 128.2 108.875) (end 131.753397 108.875) (width 0.25) (layer "B.Cu") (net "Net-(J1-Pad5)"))
 (segment (start 132.328238 109.449841) (end 132.328238 114.308172) (width 0.25) (layer "B.Cu") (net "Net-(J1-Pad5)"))
 (segment (start 121.164001 127.600002) (end 116.695001 127.600002) (width 0.25) (layer "B.Cu") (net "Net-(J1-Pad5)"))
 (segment (start 121.775001 126.989002) (end 121.164001 127.600002) (width 0.25) (layer "B.Cu") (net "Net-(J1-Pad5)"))
 (segment (start 131.753397 108.875) (end 132.328238 109.449841) (width 0.25) (layer "B.Cu") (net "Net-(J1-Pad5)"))
 (segment (start 121.150928 124.299072) (end 121.65 123.8) (width 0.25) (layer "F.Cu") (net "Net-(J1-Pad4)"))
 (segment (start 124.5 108.94) (end 124.6 108.94) (width 0.25) (layer "F.Cu") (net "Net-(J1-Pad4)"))
 (segment (start 115.4 106.6) (end 114.619981 105.819981) (width 0.25) (layer "F.Cu") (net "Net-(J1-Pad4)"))
 (segment (start 115.800001 122.561411) (end 108.55001 115.31142) (width 0.25) (layer "F.Cu") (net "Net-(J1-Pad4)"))
 (segment (start 128.6 118) (end 123.2 118) (width 0.25) (layer "F.Cu") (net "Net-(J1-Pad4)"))
 (segment (start 108.499971 115.261381) (end 108.55001 115.31142) (width 0.25) (layer "F.Cu") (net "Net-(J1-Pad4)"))
 (segment (start 124.81 109.6) (end 127.8 109.6) (width 0.25) (layer "F.Cu") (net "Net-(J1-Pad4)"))
 (segment (start 114.619981 105.819981) (end 109.543099 105.819981) (width 0.25) (layer "F.Cu") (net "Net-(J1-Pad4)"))
 (segment (start 109.543099 105.819981) (end 108.499971 106.863109) (width 0.25) (layer "F.Cu") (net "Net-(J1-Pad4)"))
 (segment (start 116.2 123.4) (end 115.800001 123.000001) (width 0.25) (layer "F.Cu") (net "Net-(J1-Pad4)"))
 (segment (start 124.6 109.39) (end 124.81 109.6) (width 0.25) (layer "F.Cu") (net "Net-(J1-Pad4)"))
 (segment (start 119.235001 125.25) (end 120.2 125.25) (width 0.25) (layer "F.Cu") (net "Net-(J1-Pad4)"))
 (segment (start 127.8 109.6) (end 129.20949 109.6) (width 0.25) (layer "F.Cu") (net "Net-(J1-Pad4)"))
 (segment (start 118.06 126.425001) (end 119.235001 125.25) (width 0.25) (layer "F.Cu") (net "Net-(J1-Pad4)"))
 (segment (start 130 109.72001) (end 130.52001 109.72001) (width 0.25) (layer "F.Cu") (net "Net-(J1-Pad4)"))
 (segment (start 120.2 125.25) (end 121.150928 124.299072) (width 0.25) (layer "F.Cu") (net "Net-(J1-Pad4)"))
 (segment (start 108.499971 106.863109) (end 108.499971 115.261381) (width 0.25) (layer "F.Cu") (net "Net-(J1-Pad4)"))
 (segment (start 129.20949 109.6) (end 129.3295 109.72001) (width 0.25) (layer "F.Cu") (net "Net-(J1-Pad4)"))
 (segment (start 131 115.6) (end 128.6 118) (width 0.25) (layer "F.Cu") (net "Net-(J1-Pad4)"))
 (segment (start 115.4 107.05) (end 115.4 106.6) (width 0.25) (layer "F.Cu") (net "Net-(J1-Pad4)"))
 (segment (start 124.6 108.94) (end 124.6 109.39) (width 0.25) (layer "F.Cu") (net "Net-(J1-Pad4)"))
 (segment (start 130.52001 109.72001) (end 131 110.2) (width 0.25) (layer "F.Cu") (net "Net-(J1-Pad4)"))
 (segment (start 129.3295 109.72001) (end 130 109.72001) (width 0.25) (layer "F.Cu") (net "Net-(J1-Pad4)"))
 (segment (start 115.800001 123.000001) (end 115.800001 122.561411) (width 0.25) (layer "F.Cu") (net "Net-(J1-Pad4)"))
 (segment (start 108.55001 115.31142) (end 108.55001 115.299971) (width 0.25) (layer "F.Cu") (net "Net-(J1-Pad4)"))
 (segment (start 131 110.2) (end 131 115.6) (width 0.25) (layer "F.Cu") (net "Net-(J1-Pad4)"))
 (segment (start 115.4 107.05) (end 115.5 107.05) (width 0.25) (layer "F.Cu") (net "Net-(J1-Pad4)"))
 (via (at 123.2 118) (size 0.8) (drill 0.4) (layers "F.Cu" "B.Cu") (capping no) (covering (front no) (back no))
  (plugging (front no) (back no)) (filling no) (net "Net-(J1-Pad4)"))
 (via (at 116.2 123.4) (size 0.8) (drill 0.4) (layers "F.Cu" "B.Cu") (capping no) (covering (front no) (back no))
  (plugging (front no) (back no)) (filling no) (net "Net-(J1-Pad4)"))
 (segment (start 116.2 123.4) (end 118.06 125.26) (width 0.25) (layer "B.Cu") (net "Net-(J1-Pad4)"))
 (segment (start 120.887317 119.746998) (end 120.6 119.746998) (width 0.25) (layer "B.Cu") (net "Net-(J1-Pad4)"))
 (segment (start 118.06 125.26) (end 118.06 126.425001) (width 0.25) (layer "B.Cu") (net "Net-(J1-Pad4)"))
 (segment (start 123.2 118) (end 122.634315 118) (width 0.25) (layer "B.Cu") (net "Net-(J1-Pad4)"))
 (segment (start 122.634315 118) (end 120.887317 119.746998) (width 0.25) (layer "B.Cu") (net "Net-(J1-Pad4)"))
 (segment (start 118.06 122.286998) (end 120.6 119.746998) (width 0.25) (layer "B.Cu") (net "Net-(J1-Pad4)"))
 (segment (start 118.06 126.425001) (end 118.06 122.286998) (width 0.25) (layer "B.Cu") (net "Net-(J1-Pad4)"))
 (segment (start 121.65 121.8) (end 119.63 121.8) (width 0.25) (layer "F.Cu") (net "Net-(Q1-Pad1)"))
 (segment (start 119.63 121.8) (end 119.6 121.77) (width 0.25) (layer "F.Cu") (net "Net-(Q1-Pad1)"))
 (segment (start 119.6 116.494988) (end 117.6 118.494988) (width 0.25) (layer "F.Cu") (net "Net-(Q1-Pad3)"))
 (segment (start 117.6 120.17) (end 117.6 120.82) (width 0.25) (layer "F.Cu") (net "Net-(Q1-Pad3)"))
 (segment (start 120 111.4) (end 119.6 111.8) (width 0.25) (layer "F.Cu") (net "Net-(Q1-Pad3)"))
 (segment (start 120 109.4825) (end 120 111.4) (width 0.25) (layer "F.Cu") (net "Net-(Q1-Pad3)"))
 (segment (start 117.6 118.494988) (end 117.6 120.17) (width 0.25) (layer "F.Cu") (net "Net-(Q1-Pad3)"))
 (segment (start 119.6 111.8) (end 119.6 116.494988) (width 0.25) (layer "F.Cu") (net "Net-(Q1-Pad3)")))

